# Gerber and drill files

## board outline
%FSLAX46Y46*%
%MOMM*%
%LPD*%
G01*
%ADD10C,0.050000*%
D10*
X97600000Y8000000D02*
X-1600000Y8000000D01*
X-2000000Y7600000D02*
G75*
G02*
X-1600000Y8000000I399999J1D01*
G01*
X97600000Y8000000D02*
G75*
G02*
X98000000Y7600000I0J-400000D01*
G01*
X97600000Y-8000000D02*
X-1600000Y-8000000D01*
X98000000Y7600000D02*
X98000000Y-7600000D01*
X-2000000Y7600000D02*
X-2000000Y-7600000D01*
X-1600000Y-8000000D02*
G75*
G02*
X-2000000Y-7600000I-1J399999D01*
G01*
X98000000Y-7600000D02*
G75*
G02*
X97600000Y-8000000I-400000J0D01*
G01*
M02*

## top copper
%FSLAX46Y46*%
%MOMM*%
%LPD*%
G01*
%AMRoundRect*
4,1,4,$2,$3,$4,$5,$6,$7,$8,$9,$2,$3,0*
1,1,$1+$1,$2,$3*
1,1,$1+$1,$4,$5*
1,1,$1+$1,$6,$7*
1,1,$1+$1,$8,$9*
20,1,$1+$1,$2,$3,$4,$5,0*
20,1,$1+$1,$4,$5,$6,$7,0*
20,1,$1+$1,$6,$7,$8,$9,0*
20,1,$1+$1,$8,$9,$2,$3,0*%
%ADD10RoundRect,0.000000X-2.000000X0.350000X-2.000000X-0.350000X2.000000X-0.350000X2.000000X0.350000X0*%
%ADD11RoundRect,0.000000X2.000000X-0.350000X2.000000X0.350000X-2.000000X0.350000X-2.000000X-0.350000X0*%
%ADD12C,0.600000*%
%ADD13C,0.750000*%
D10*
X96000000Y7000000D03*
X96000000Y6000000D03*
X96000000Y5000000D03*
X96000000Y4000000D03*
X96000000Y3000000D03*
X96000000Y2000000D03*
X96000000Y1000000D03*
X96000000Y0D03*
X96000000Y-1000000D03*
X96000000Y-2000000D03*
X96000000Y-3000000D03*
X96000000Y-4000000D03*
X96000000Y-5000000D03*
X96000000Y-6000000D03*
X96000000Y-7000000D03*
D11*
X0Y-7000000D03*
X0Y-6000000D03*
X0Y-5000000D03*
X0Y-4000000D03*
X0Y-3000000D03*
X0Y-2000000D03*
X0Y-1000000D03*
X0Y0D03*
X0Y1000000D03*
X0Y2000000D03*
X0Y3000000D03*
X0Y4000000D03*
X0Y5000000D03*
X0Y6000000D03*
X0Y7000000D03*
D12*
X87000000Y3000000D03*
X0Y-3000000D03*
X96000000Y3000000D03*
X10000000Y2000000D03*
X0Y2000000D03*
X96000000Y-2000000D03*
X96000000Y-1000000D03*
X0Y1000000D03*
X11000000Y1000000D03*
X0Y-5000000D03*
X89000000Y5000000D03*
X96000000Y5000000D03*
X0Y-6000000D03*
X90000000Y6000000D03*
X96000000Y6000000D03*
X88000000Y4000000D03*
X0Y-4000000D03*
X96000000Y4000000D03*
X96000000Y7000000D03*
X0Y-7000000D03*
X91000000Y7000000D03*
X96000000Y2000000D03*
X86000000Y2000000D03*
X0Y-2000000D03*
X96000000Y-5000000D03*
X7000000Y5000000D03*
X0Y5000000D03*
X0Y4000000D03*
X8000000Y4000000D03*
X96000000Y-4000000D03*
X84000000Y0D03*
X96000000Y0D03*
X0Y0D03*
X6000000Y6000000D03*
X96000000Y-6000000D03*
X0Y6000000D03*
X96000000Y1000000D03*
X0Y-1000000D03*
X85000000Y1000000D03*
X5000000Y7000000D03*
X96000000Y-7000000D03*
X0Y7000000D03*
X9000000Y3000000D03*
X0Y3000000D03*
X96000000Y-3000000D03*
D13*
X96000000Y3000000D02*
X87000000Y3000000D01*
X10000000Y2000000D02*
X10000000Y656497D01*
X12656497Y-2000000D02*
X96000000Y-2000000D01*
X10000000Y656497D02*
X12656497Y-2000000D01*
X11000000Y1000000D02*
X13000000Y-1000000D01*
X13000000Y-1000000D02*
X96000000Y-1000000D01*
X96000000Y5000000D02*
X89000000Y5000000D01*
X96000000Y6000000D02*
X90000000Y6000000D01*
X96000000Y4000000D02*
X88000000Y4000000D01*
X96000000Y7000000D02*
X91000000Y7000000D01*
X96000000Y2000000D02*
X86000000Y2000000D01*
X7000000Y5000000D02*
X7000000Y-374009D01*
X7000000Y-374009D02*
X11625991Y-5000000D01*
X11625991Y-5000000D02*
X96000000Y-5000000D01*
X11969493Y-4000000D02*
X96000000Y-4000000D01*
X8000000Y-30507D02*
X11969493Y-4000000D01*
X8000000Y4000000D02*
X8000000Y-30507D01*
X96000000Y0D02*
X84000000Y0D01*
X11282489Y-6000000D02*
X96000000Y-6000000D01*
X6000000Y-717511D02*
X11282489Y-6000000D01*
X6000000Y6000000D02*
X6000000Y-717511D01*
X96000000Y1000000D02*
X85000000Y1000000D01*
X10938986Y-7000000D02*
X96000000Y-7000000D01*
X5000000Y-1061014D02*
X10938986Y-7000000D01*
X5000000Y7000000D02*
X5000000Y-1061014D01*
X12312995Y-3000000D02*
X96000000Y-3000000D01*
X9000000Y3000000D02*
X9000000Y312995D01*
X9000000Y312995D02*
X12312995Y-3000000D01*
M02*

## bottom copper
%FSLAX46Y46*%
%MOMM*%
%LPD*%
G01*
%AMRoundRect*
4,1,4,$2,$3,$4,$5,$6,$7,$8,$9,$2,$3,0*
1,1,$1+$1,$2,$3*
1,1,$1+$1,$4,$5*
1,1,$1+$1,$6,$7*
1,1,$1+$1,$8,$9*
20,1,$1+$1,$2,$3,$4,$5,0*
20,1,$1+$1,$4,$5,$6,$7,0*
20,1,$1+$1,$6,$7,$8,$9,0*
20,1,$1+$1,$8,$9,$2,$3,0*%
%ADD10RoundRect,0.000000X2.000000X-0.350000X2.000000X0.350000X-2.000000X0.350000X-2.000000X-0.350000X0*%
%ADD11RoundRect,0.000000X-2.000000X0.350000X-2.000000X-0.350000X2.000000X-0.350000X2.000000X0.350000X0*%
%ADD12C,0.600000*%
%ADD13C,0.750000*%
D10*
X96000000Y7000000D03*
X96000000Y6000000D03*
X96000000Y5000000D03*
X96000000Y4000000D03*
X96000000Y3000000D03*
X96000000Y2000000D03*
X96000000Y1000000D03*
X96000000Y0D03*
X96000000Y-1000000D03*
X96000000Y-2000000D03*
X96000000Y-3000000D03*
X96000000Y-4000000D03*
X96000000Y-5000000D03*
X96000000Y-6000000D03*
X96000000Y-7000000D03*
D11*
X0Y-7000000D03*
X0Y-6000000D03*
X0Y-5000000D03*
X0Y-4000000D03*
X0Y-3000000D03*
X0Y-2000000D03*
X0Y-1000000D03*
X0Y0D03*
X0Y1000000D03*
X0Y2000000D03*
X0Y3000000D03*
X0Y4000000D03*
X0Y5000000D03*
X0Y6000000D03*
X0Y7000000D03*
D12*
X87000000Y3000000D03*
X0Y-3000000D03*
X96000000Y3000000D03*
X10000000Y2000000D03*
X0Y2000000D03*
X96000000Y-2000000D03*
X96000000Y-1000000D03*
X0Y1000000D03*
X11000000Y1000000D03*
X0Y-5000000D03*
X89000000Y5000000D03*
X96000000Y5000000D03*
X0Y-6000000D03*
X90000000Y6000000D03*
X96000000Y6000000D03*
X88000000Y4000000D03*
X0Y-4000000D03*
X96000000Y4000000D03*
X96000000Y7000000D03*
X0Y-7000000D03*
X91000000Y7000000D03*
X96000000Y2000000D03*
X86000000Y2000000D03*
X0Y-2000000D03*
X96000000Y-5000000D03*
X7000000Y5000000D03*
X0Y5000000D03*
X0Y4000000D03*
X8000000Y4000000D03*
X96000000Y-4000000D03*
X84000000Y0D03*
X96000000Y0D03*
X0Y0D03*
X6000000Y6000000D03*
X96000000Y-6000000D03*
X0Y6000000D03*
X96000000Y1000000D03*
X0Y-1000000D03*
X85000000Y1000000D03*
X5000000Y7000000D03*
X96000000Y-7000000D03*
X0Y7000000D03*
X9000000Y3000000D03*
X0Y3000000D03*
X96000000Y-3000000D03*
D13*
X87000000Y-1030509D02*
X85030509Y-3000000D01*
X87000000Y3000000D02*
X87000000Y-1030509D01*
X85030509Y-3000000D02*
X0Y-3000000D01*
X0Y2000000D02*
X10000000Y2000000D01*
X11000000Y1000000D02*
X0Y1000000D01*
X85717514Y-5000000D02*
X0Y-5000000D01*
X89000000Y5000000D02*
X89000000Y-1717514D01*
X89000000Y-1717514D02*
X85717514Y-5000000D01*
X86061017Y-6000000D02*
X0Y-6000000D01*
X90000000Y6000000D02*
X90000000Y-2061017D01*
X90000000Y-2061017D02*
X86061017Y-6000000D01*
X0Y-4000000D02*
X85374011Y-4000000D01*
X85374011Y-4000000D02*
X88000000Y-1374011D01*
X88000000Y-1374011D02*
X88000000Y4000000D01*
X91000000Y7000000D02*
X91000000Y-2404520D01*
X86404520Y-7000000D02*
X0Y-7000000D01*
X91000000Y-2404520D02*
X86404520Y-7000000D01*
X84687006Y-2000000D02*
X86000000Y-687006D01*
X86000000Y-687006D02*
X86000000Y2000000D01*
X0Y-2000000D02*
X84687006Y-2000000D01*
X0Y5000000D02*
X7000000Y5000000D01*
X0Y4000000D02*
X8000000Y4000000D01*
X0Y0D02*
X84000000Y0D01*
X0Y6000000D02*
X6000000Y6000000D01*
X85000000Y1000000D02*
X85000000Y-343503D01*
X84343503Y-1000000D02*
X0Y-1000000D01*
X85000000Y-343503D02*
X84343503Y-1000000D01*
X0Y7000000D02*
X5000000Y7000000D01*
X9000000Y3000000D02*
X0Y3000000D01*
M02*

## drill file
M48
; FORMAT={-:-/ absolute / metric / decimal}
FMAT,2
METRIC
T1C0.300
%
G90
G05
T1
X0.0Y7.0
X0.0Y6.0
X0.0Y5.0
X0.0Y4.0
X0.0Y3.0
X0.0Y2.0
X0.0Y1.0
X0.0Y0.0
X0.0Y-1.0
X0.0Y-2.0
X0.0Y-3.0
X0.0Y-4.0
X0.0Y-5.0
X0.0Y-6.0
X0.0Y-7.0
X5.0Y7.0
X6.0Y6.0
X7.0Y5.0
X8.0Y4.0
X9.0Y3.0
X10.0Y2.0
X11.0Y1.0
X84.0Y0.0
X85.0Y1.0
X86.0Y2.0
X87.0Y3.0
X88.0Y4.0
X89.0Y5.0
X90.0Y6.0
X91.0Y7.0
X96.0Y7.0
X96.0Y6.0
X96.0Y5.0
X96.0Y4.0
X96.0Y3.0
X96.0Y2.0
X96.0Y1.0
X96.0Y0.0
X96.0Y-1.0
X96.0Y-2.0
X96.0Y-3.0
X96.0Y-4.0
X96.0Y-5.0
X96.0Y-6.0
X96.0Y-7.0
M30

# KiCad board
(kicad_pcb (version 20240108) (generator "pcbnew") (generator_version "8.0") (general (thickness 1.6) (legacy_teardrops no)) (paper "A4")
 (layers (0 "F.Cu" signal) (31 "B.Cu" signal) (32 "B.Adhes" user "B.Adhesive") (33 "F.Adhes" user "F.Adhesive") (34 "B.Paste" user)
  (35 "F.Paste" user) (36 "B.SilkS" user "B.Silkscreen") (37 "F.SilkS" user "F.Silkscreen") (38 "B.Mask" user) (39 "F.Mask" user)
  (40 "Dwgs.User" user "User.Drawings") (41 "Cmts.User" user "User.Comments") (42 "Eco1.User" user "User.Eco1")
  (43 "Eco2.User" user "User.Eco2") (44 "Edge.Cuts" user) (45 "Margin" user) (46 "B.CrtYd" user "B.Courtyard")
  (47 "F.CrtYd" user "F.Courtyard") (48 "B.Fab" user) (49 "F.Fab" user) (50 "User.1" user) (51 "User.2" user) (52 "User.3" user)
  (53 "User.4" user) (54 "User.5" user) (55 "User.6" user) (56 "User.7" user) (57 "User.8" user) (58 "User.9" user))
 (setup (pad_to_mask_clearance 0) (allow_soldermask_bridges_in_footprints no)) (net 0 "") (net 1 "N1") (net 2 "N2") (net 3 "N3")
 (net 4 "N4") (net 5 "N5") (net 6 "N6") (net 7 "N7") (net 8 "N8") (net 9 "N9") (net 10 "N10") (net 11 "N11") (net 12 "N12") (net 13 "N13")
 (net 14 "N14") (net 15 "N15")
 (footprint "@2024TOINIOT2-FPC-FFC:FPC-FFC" (layer "F.Cu") (at 96 0 -90)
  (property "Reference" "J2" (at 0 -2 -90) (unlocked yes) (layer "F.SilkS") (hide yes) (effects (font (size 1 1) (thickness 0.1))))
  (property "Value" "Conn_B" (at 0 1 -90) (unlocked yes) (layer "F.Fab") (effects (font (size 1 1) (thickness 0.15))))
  (pad "1" smd roundrect (at -7 0 270) (size 0.7 4) (layers "F.Cu" "F.Paste" "B.SilkS" "F.Mask") (roundrect_rratio 0) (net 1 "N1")
   (thermal_bridge_angle 45))
  (pad "1" smd roundrect (at -7 0 90) (size 0.7 4) (layers "B.Cu" "B.Paste" "F.SilkS" "B.Mask") (roundrect_rratio 0) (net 1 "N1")
   (thermal_bridge_angle 45))
  (pad "2" smd roundrect (at -6 0 270) (size 0.7 4) (layers "F.Cu" "F.Paste" "B.SilkS" "F.Mask") (roundrect_rratio 0) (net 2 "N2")
   (thermal_bridge_angle 45))
  (pad "2" smd roundrect (at -6 0 90) (size 0.7 4) (layers "B.Cu" "B.Paste" "F.SilkS" "B.Mask") (roundrect_rratio 0) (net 2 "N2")
   (thermal_bridge_angle 45))
  (pad "3" smd roundrect (at -5 0 270) (size 0.7 4) (layers "F.Cu" "F.Paste" "B.SilkS" "F.Mask") (roundrect_rratio 0) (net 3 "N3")
   (thermal_bridge_angle 45))
  (pad "3" smd roundrect (at -5 0 90) (size 0.7 4) (layers "B.Cu" "B.Paste" "F.SilkS" "B.Mask") (roundrect_rratio 0) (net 3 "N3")
   (thermal_bridge_angle 45))
  (pad "4" smd roundrect (at -4 0 270) (size 0.7 4) (layers "F.Cu" "F.Paste" "B.SilkS" "F.Mask") (roundrect_rratio 0) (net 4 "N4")
   (thermal_bridge_angle 45))
  (pad "4" smd roundrect (at -4 0 90) (size 0.7 4) (layers "B.Cu" "B.Paste" "F.SilkS" "B.Mask") (roundrect_rratio 0) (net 4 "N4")
   (thermal_bridge_angle 45))
  (pad "5" smd roundrect (at -3 0 270) (size 0.7 4) (layers "F.Cu" "F.Paste" "B.SilkS" "F.Mask") (roundrect_rratio 0) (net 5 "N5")
   (thermal_bridge_angle 45))
  (pad "5" smd roundrect (at -3 0 90) (size 0.7 4) (layers "B.Cu" "B.Paste" "F.SilkS" "B.Mask") (roundrect_rratio 0) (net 5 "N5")
   (thermal_bridge_angle 45))
  (pad "6" smd roundrect (at -2 0 270) (size 0.7 4) (layers "F.Cu" "F.Paste" "B.SilkS" "F.Mask") (roundrect_rratio 0) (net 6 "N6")
   (thermal_bridge_angle 45))
  (pad "6" smd roundrect (at -2 0 90) (size 0.7 4) (layers "B.Cu" "B.Paste" "F.SilkS" "B.Mask") (roundrect_rratio 0) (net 6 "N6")
   (thermal_bridge_angle 45))
  (pad "7" smd roundrect (at -1 0 270) (size 0.7 4) (layers "F.Cu" "F.Paste" "B.SilkS" "F.Mask") (roundrect_rratio 0) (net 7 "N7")
   (thermal_bridge_angle 45))
  (pad "7" smd roundrect (at -1 0 90) (size 0.7 4) (layers "B.Cu" "B.Paste" "F.SilkS" "B.Mask") (roundrect_rratio 0) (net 7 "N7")
   (thermal_bridge_angle 45))
  (pad "8" smd roundrect (at 0 0 270) (size 0.7 4) (layers "F.Cu" "F.Paste" "B.SilkS" "F.Mask") (roundrect_rratio 0) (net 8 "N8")
   (thermal_bridge_angle 45))
  (pad "8" smd roundrect (at 0 0 90) (size 0.7 4) (layers "B.Cu" "B.Paste" "F.SilkS" "B.Mask") (roundrect_rratio 0) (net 8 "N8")
   (thermal_bridge_angle 45))
  (pad "9" smd roundrect (at 1 0 270) (size 0.7 4) (layers "F.Cu" "F.Paste" "B.SilkS" "F.Mask") (roundrect_rratio 0) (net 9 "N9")
   (thermal_bridge_angle 45))
  (pad "9" smd roundrect (at 1 0 90) (size 0.7 4) (layers "B.Cu" "B.Paste" "F.SilkS" "B.Mask") (roundrect_rratio 0) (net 9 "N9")
   (thermal_bridge_angle 45))
  (pad "10" smd roundrect (at 2 0 270) (size 0.7 4) (layers "F.Cu" "F.Paste" "B.SilkS" "F.Mask") (roundrect_rratio 0) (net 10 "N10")
   (thermal_bridge_angle 45))
  (pad "10" smd roundrect (at 2 0 90) (size 0.7 4) (layers "B.Cu" "B.Paste" "F.SilkS" "B.Mask") (roundrect_rratio 0) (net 10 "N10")
   (thermal_bridge_angle 45))
  (pad "11" smd roundrect (at 3 0 270) (size 0.7 4) (layers "F.Cu" "F.Paste" "B.SilkS" "F.Mask") (roundrect_rratio 0) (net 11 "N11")
   (thermal_bridge_angle 45))
  (pad "11" smd roundrect (at 3 0 90) (size 0.7 4) (layers "B.Cu" "B.Paste" "F.SilkS" "B.Mask") (roundrect_rratio 0) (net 11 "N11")
   (thermal_bridge_angle 45))
  (pad "12" smd roundrect (at 4 0 270) (size 0.7 4) (layers "F.Cu" "F.Paste" "B.SilkS" "F.Mask") (roundrect_rratio 0) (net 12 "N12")
   (thermal_bridge_angle 45))
  (pad "12" smd roundrect (at 4 0 90) (size 0.7 4) (layers "B.Cu" "B.Paste" "F.SilkS" "B.Mask") (roundrect_rratio 0) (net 12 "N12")
   (thermal_bridge_angle 45))
  (pad "13" smd roundrect (at 5 0 270) (size 0.7 4) (layers "F.Cu" "F.Paste" "B.SilkS" "F.Mask") (roundrect_rratio 0) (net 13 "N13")
   (thermal_bridge_angle 45))
  (pad "13" smd roundrect (at 5 0 90) (size 0.7 4) (layers "B.Cu" "B.Paste" "F.SilkS" "B.Mask") (roundrect_rratio 0) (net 13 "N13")
   (thermal_bridge_angle 45))
  (pad "14" smd roundrect (at 6 0 270) (size 0.7 4) (layers "F.Cu" "F.Paste" "B.SilkS" "F.Mask") (roundrect_rratio 0) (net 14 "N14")
   (thermal_bridge_angle 45))
  (pad "14" smd roundrect (at 6 0 90) (size 0.7 4) (layers "B.Cu" "B.Paste" "F.SilkS" "B.Mask") (roundrect_rratio 0) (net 14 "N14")
   (thermal_bridge_angle 45))
  (pad "15" smd roundrect (at 7 0 270) (size 0.7 4) (layers "F.Cu" "F.Paste" "B.SilkS" "F.Mask") (roundrect_rratio 0) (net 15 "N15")
   (thermal_bridge_angle 45))
  (pad "15" smd roundrect (at 7 0 90) (size 0.7 4) (layers "B.Cu" "B.Paste" "F.SilkS" "B.Mask") (roundrect_rratio 0) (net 15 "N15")
   (thermal_bridge_angle 45)))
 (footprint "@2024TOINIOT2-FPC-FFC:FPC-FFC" (layer "F.Cu") (at 0 0 90)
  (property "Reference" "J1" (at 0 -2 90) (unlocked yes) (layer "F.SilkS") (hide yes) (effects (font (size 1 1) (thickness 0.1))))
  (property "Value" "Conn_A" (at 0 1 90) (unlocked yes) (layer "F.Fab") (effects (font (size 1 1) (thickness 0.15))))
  (pad "1" smd roundrect (at -7 0 90) (size 0.7 4) (layers "F.Cu" "F.Paste" "B.SilkS" "F.Mask") (roundrect_rratio 0) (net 1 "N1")
   (thermal_bridge_angle 45))
  (pad "1" smd roundrect (at -7 0 270) (size 0.7 4) (layers "B.Cu" "B.Paste" "F.SilkS" "B.Mask") (roundrect_rratio 0) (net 1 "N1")
   (thermal_bridge_angle 45))
  (pad "2" smd roundrect (at -6 0 90) (size 0.7 4) (layers "F.Cu" "F.Paste" "B.SilkS" "F.Mask") (roundrect_rratio 0) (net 2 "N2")
   (thermal_bridge_angle 45))
  (pad "2" smd roundrect (at -6 0 270) (size 0.7 4) (layers "B.Cu" "B.Paste" "F.SilkS" "B.Mask") (roundrect_rratio 0) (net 2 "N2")
   (thermal_bridge_angle 45))
  (pad "3" smd roundrect (at -5 0 90) (size 0.7 4) (layers "F.Cu" "F.Paste" "B.SilkS" "F.Mask") (roundrect_rratio 0) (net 3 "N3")
   (thermal_bridge_angle 45))
  (pad "3" smd roundrect (at -5 0 270) (size 0.7 4) (layers "B.Cu" "B.Paste" "F.SilkS" "B.Mask") (roundrect_rratio 0) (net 3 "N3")
   (thermal_bridge_angle 45))
  (pad "4" smd roundrect (at -4 0 90) (size 0.7 4) (layers "F.Cu" "F.Paste" "B.SilkS" "F.Mask") (roundrect_rratio 0) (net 4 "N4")
   (thermal_bridge_angle 45))
  (pad "4" smd roundrect (at -4 0 270) (size 0.7 4) (layers "B.Cu" "B.Paste" "F.SilkS" "B.Mask") (roundrect_rratio 0) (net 4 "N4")
   (thermal_bridge_angle 45))
  (pad "5" smd roundrect (at -3 0 90) (size 0.7 4) (layers "F.Cu" "F.Paste" "B.SilkS" "F.Mask") (roundrect_rratio 0) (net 5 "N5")
   (thermal_bridge_angle 45))
  (pad "5" smd roundrect (at -3 0 270) (size 0.7 4) (layers "B.Cu" "B.Paste" "F.SilkS" "B.Mask") (roundrect_rratio 0) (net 5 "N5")
   (thermal_bridge_angle 45))
  (pad "6" smd roundrect (at -2 0 90) (size 0.7 4) (layers "F.Cu" "F.Paste" "B.SilkS" "F.Mask") (roundrect_rratio 0) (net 6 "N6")
   (thermal_bridge_angle 45))
  (pad "6" smd roundrect (at -2 0 270) (size 0.7 4) (layers "B.Cu" "B.Paste" "F.SilkS" "B.Mask") (roundrect_rratio 0) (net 6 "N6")
   (thermal_bridge_angle 45))
  (pad "7" smd roundrect (at -1 0 90) (size 0.7 4) (layers "F.Cu" "F.Paste" "B.SilkS" "F.Mask") (roundrect_rratio 0) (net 7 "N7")
   (thermal_bridge_angle 45))
  (pad "7" smd roundrect (at -1 0 270) (size 0.7 4) (layers "B.Cu" "B.Paste" "F.SilkS" "B.Mask") (roundrect_rratio 0) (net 7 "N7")
   (thermal_bridge_angle 45))
  (pad "8" smd roundrect (at 0 0 90) (size 0.7 4) (layers "F.Cu" "F.Paste" "B.SilkS" "F.Mask") (roundrect_rratio 0) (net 8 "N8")
   (thermal_bridge_angle 45))
  (pad "8" smd roundrect (at 0 0 270) (size 0.7 4) (layers "B.Cu" "B.Paste" "F.SilkS" "B.Mask") (roundrect_rratio 0) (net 8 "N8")
   (thermal_bridge_angle 45))
  (pad "9" smd roundrect (at 1 0 90) (size 0.7 4) (layers "F.Cu" "F.Paste" "B.SilkS" "F.Mask") (roundrect_rratio 0) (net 9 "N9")
   (thermal_bridge_angle 45))
  (pad "9" smd roundrect (at 1 0 270) (size 0.7 4) (layers "B.Cu" "B.Paste" "F.SilkS" "B.Mask") (roundrect_rratio 0) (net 9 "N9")
   (thermal_bridge_angle 45))
  (pad "10" smd roundrect (at 2 0 90) (size 0.7 4) (layers "F.Cu" "F.Paste" "B.SilkS" "F.Mask") (roundrect_rratio 0) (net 10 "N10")
   (thermal_bridge_angle 45))
  (pad "10" smd roundrect (at 2 0 270) (size 0.7 4) (layers "B.Cu" "B.Paste" "F.SilkS" "B.Mask") (roundrect_rratio 0) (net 10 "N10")
   (thermal_bridge_angle 45))
  (pad "11" smd roundrect (at 3 0 90) (size 0.7 4) (layers "F.Cu" "F.Paste" "B.SilkS" "F.Mask") (roundrect_rratio 0) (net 11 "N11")
   (thermal_bridge_angle 45))
  (pad "11" smd roundrect (at 3 0 270) (size 0.7 4) (layers "B.Cu" "B.Paste" "F.SilkS" "B.Mask") (roundrect_rratio 0) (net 11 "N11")
   (thermal_bridge_angle 45))
  (pad "12" smd roundrect (at 4 0 90) (size 0.7 4) (layers "F.Cu" "F.Paste" "B.SilkS" "F.Mask") (roundrect_rratio 0) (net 12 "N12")
   (thermal_bridge_angle 45))
  (pad "12" smd roundrect (at 4 0 270) (size 0.7 4) (layers "B.Cu" "B.Paste" "F.SilkS" "B.Mask") (roundrect_rratio 0) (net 12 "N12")
   (thermal_bridge_angle 45))
  (pad "13" smd roundrect (at 5 0 90) (size 0.7 4) (layers "F.Cu" "F.Paste" "B.SilkS" "F.Mask") (roundrect_rratio 0) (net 13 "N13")
   (thermal_bridge_angle 45))
  (pad "13" smd roundrect (at 5 0 270) (size 0.7 4) (layers "B.Cu" "B.Paste" "F.SilkS" "B.Mask") (roundrect_rratio 0) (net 13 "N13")
   (thermal_bridge_angle 45))
  (pad "14" smd roundrect (at 6 0 90) (size 0.7 4) (layers "F.Cu" "F.Paste" "B.SilkS" "F.Mask") (roundrect_rratio 0) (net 14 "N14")
   (thermal_bridge_angle 45))
  (pad "14" smd roundrect (at 6 0 270) (size 0.7 4) (layers "B.Cu" "B.Paste" "F.SilkS" "B.Mask") (roundrect_rratio 0) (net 14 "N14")
   (thermal_bridge_angle 45))
  (pad "15" smd roundrect (at 7 0 90) (size 0.7 4) (layers "F.Cu" "F.Paste" "B.SilkS" "F.Mask") (roundrect_rratio 0) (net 15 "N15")
   (thermal_bridge_angle 45))
  (pad "15" smd roundrect (at 7 0 270) (size 0.7 4) (layers "B.Cu" "B.Paste" "F.SilkS" "B.Mask") (roundrect_rratio 0) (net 15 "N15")
   (thermal_bridge_angle 45)))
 (gr_line (start 97.6 -8) (end -1.6 -8) (stroke (width 0.05) (type default)) (layer "Edge.Cuts"))
 (gr_arc (start -2 -7.6) (mid -1.882843 -7.882843) (end -1.6 -8) (stroke (width 0.05) (type default)) (layer "Edge.Cuts"))
 (gr_arc (start 97.6 -8) (mid 97.882843 -7.882843) (end 98 -7.6) (stroke (width 0.05) (type default)) (layer "Edge.Cuts"))
 (gr_line (start 97.6 8) (end -1.6 8) (stroke (width 0.05) (type default)) (layer "Edge.Cuts"))
 (gr_line (start 98 -7.6) (end 98 7.6) (stroke (width 0.05) (type default)) (layer "Edge.Cuts"))
 (gr_line (start -2 -7.6) (end -2 7.6) (stroke (width 0.05) (type default)) (layer "Edge.Cuts"))
 (gr_arc (start -1.6 8) (mid -1.882843 7.882843) (end -2 7.6) (stroke (width 0.05) (type default)) (layer "Edge.Cuts"))
 (gr_arc (start 98 7.6) (mid 97.882843 7.882843) (end 97.6 8) (stroke (width 0.05) (type default)) (layer "Edge.Cuts"))
 (segment (start 96 -3) (end 87 -3) (width 0.75) (layer "F.Cu") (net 5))
 (via (at 87 -3) (size 0.6) (drill 0.3) (layers "F.Cu" "B.Cu") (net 5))
 (via (at 0 3) (size 0.6) (drill 0.3) (layers "F.Cu" "B.Cu") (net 5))
 (via (at 96 -3) (size 0.6) (drill 0.3) (layers "F.Cu" "B.Cu") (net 5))
 (segment (start 87 1.030509) (end 85.030509 3) (width 0.75) (layer "B.Cu") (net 5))
 (segment (start 87 -3) (end 87 1.030509) (width 0.75) (layer "B.Cu") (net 5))
 (segment (start 85.030509 3) (end 0 3) (width 0.75) (layer "B.Cu") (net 5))
 (segment (start 10 -2) (end 10 -0.656497) (width 0.75) (layer "F.Cu") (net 10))
 (segment (start 12.656497 2) (end 96 2) (width 0.75) (layer "F.Cu") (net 10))
 (segment (start 10 -0.656497) (end 12.656497 2) (width 0.75) (layer "F.Cu") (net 10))
 (via (at 10 -2) (size 0.6) (drill 0.3) (layers "F.Cu" "B.Cu") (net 10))
 (via (at 0 -2) (size 0.6) (drill 0.3) (layers "F.Cu" "B.Cu") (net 10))
 (via (at 96 2) (size 0.6) (drill 0.3) (layers "F.Cu" "B.Cu") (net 10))
 (segment (start 0 -2) (end 10 -2) (width 0.75) (layer "B.Cu") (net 10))
 (segment (start 11 -1) (end 13 1) (width 0.75) (layer "F.Cu") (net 9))
 (segment (start 13 1) (end 96 1) (width 0.75) (layer "F.Cu") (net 9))
 (via (at 96 1) (size 0.6) (drill 0.3) (layers "F.Cu" "B.Cu") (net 9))
 (via (at 0 -1) (size 0.6) (drill 0.3) (layers "F.Cu" "B.Cu") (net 9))
 (via (at 11 -1) (size 0.6) (drill 0.3) (layers "F.Cu" "B.Cu") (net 9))
 (segment (start 11 -1) (end 0 -1) (width 0.75) (layer "B.Cu") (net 9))
 (segment (start 96 -5) (end 89 -5) (width 0.75) (layer "F.Cu") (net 3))
 (via (at 0 5) (size 0.6) (drill 0.3) (layers "F.Cu" "B.Cu") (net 3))
 (via (at 89 -5) (size 0.6) (drill 0.3) (layers "F.Cu" "B.Cu") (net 3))
 (via (at 96 -5) (size 0.6) (drill 0.3) (layers "F.Cu" "B.Cu") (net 3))
 (segment (start 85.717514 5) (end 0 5) (width 0.75) (layer "B.Cu") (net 3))
 (segment (start 89 -5) (end 89 1.717514) (width 0.75) (layer "B.Cu") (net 3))
 (segment (start 89 1.717514) (end 85.717514 5) (width 0.75) (layer "B.Cu") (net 3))
 (segment (start 96 -6) (end 90 -6) (width 0.75) (layer "F.Cu") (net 2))
 (via (at 0 6) (size 0.6) (drill 0.3) (layers "F.Cu" "B.Cu") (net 2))
 (via (at 90 -6) (size 0.6) (drill 0.3) (layers "F.Cu" "B.Cu") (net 2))
 (via (at 96 -6) (size 0.6) (drill 0.3) (layers "F.Cu" "B.Cu") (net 2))
 (segment (start 86.061017 6) (end 0 6) (width 0.75) (layer "B.Cu") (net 2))
 (segment (start 90 -6) (end 90 2.061017) (width 0.75) (layer "B.Cu") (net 2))
 (segment (start 90 2.061017) (end 86.061017 6) (width 0.75) (layer "B.Cu") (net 2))
 (segment (start 96 -4) (end 88 -4) (width 0.75) (layer "F.Cu") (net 4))
 (via (at 88 -4) (size 0.6) (drill 0.3) (layers "F.Cu" "B.Cu") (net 4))
 (via (at 0 4) (size 0.6) (drill 0.3) (layers "F.Cu" "B.Cu") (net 4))
 (via (at 96 -4) (size 0.6) (drill 0.3) (layers "F.Cu" "B.Cu") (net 4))
 (segment (start 0 4) (end 85.374011 4) (width 0.75) (layer "B.Cu") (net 4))
 (segment (start 85.374011 4) (end 88 1.374011) (width 0.75) (layer "B.Cu") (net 4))
 (segment (start 88 1.374011) (end 88 -4) (width 0.75) (layer "B.Cu") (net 4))
 (segment (start 96 -7) (end 91 -7) (width 0.75) (layer "F.Cu") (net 1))
 (via (at 96 -7) (size 0.6) (drill 0.3) (layers "F.Cu" "B.Cu") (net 1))
 (via (at 0 7) (size 0.6) (drill 0.3) (layers "F.Cu" "B.Cu") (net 1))
 (via (at 91 -7) (size 0.6) (drill 0.3) (layers "F.Cu" "B.Cu") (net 1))
 (segment (start 91 -7) (end 91 2.40452) (width 0.75) (layer "B.Cu") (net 1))
 (segment (start 86.40452 7) (end 0 7) (width 0.75) (layer "B.Cu") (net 1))
 (segment (start 91 2.40452) (end 86.40452 7) (width 0.75) (layer "B.Cu") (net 1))
 (segment (start 96 -2) (end 86 -2) (width 0.75) (layer "F.Cu") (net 6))
 (via (at 96 -2) (size 0.6) (drill 0.3) (layers "F.Cu" "B.Cu") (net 6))
 (via (at 86 -2) (size 0.6) (drill 0.3) (layers "F.Cu" "B.Cu") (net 6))
 (via (at 0 2) (size 0.6) (drill 0.3) (layers "F.Cu" "B.Cu") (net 6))
 (segment (start 84.687006 2) (end 86 0.687006) (width 0.75) (layer "B.Cu") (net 6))
 (segment (start 86 0.687006) (end 86 -2) (width 0.75) (layer "B.Cu") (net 6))
 (segment (start 0 2) (end 84.687006 2) (width 0.75) (layer "B.Cu") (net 6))
 (segment (start 7 -5) (end 7 0.374009) (width 0.75) (layer "F.Cu") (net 13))
 (segment (start 7 0.374009) (end 11.625991 5) (width 0.75) (layer "F.Cu") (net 13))
 (segment (start 11.625991 5) (end 96 5) (width 0.75) (layer "F.Cu") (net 13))
 (via (at 96 5) (size 0.6) (drill 0.3) (layers "F.Cu" "B.Cu") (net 13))
 (via (at 7 -5) (size 0.6) (drill 0.3) (layers "F.Cu" "B.Cu") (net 13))
 (via (at 0 -5) (size 0.6) (drill 0.3) (layers "F.Cu" "B.Cu") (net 13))
 (segment (start 0 -5) (end 7 -5) (width 0.75) (layer "B.Cu") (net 13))
 (segment (start 11.969493 4) (end 96 4) (width 0.75) (layer "F.Cu") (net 12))
 (segment (start 8 0.030507) (end 11.969493 4) (width 0.75) (layer "F.Cu") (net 12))
 (segment (start 8 -4) (end 8 0.030507) (width 0.75) (layer "F.Cu") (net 12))
 (via (at 0 -4) (size 0.6) (drill 0.3) (layers "F.Cu" "B.Cu") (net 12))
 (via (at 8 -4) (size 0.6) (drill 0.3) (layers "F.Cu" "B.Cu") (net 12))
 (via (at 96 4) (size 0.6) (drill 0.3) (layers "F.Cu" "B.Cu") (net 12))
 (segment (start 0 -4) (end 8 -4) (width 0.75) (layer "B.Cu") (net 12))
 (segment (start 96 0) (end 84 0) (width 0.75) (layer "F.Cu") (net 8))
 (via (at 84 0) (size 0.6) (drill 0.3) (layers "F.Cu" "B.Cu") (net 8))
 (via (at 96 0) (size 0.6) (drill 0.3) (layers "F.Cu" "B.Cu") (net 8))
 (via (at 0 0) (size 0.6) (drill 0.3) (layers "F.Cu" "B.Cu") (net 8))
 (segment (start 0 0) (end 84 0) (width 0.75) (layer "B.Cu") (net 8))
 (segment (start 11.282489 6) (end 96 6) (width 0.75) (layer "F.Cu") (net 14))
 (segment (start 6 0.717511) (end 11.282489 6) (width 0.75) (layer "F.Cu") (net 14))
 (segment (start 6 -6) (end 6 0.717511) (width 0.75) (layer "F.Cu") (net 14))
 (via (at 6 -6) (size 0.6) (drill 0.3) (layers "F.Cu" "B.Cu") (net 14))
 (via (at 96 6) (size 0.6) (drill 0.3) (layers "F.Cu" "B.Cu") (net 14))
 (via (at 0 -6) (size 0.6) (drill 0.3) (layers "F.Cu" "B.Cu") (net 14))
 (segment (start 0 -6) (end 6 -6) (width 0.75) (layer "B.Cu") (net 14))
 (segment (start 96 -1) (end 85 -1) (width 0.75) (layer "F.Cu") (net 7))
 (via (at 96 -1) (size 0.6) (drill 0.3) (layers "F.Cu" "B.Cu") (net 7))
 (via (at 0 1) (size 0.6) (drill 0.3) (layers "F.Cu" "B.Cu") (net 7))
 (via (at 85 -1) (size 0.6) (drill 0.3) (layers "F.Cu" "B.Cu") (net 7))
 (segment (start 85 -1) (end 85 0.343503) (width 0.75) (layer "B.Cu") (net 7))
 (segment (start 84.343503 1) (end 0 1) (width 0.75) (layer "B.Cu") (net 7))
 (segment (start 85 0.343503) (end 84.343503 1) (width 0.75) (layer "B.Cu") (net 7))
 (segment (start 10.938986 7) (end 96 7) (width 0.75) (layer "F.Cu") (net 15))
 (segment (start 5 1.061014) (end 10.938986 7) (width 0.75) (layer "F.Cu") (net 15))
 (segment (start 5 -7) (end 5 1.061014) (width 0.75) (layer "F.Cu") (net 15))
 (via (at 5 -7) (size 0.6) (drill 0.3) (layers "F.Cu" "B.Cu") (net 15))
 (via (at 96 7) (size 0.6) (drill 0.3) (layers "F.Cu" "B.Cu") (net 15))
 (via (at 0 -7) (size 0.6) (drill 0.3) (layers "F.Cu" "B.Cu") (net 15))
 (segment (start 0 -7) (end 5 -7) (width 0.75) (layer "B.Cu") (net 15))
 (segment (start 12.312995 3) (end 96 3) (width 0.75) (layer "F.Cu") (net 11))
 (segment (start 9 -3) (end 9 -0.312995) (width 0.75) (layer "F.Cu") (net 11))
 (segment (start 9 -0.312995) (end 12.312995 3) (width 0.75) (layer "F.Cu") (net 11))
 (via (at 9 -3) (size 0.6) (drill 0.3) (layers "F.Cu" "B.Cu") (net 11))
 (via (at 0 -3) (size 0.6) (drill 0.3) (layers "F.Cu" "B.Cu") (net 11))
 (via (at 96 3) (size 0.6) (drill 0.3) (layers "F.Cu" "B.Cu") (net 11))
 (segment (start 9 -3) (end 0 -3) (width 0.75) (layer "B.Cu") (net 11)))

